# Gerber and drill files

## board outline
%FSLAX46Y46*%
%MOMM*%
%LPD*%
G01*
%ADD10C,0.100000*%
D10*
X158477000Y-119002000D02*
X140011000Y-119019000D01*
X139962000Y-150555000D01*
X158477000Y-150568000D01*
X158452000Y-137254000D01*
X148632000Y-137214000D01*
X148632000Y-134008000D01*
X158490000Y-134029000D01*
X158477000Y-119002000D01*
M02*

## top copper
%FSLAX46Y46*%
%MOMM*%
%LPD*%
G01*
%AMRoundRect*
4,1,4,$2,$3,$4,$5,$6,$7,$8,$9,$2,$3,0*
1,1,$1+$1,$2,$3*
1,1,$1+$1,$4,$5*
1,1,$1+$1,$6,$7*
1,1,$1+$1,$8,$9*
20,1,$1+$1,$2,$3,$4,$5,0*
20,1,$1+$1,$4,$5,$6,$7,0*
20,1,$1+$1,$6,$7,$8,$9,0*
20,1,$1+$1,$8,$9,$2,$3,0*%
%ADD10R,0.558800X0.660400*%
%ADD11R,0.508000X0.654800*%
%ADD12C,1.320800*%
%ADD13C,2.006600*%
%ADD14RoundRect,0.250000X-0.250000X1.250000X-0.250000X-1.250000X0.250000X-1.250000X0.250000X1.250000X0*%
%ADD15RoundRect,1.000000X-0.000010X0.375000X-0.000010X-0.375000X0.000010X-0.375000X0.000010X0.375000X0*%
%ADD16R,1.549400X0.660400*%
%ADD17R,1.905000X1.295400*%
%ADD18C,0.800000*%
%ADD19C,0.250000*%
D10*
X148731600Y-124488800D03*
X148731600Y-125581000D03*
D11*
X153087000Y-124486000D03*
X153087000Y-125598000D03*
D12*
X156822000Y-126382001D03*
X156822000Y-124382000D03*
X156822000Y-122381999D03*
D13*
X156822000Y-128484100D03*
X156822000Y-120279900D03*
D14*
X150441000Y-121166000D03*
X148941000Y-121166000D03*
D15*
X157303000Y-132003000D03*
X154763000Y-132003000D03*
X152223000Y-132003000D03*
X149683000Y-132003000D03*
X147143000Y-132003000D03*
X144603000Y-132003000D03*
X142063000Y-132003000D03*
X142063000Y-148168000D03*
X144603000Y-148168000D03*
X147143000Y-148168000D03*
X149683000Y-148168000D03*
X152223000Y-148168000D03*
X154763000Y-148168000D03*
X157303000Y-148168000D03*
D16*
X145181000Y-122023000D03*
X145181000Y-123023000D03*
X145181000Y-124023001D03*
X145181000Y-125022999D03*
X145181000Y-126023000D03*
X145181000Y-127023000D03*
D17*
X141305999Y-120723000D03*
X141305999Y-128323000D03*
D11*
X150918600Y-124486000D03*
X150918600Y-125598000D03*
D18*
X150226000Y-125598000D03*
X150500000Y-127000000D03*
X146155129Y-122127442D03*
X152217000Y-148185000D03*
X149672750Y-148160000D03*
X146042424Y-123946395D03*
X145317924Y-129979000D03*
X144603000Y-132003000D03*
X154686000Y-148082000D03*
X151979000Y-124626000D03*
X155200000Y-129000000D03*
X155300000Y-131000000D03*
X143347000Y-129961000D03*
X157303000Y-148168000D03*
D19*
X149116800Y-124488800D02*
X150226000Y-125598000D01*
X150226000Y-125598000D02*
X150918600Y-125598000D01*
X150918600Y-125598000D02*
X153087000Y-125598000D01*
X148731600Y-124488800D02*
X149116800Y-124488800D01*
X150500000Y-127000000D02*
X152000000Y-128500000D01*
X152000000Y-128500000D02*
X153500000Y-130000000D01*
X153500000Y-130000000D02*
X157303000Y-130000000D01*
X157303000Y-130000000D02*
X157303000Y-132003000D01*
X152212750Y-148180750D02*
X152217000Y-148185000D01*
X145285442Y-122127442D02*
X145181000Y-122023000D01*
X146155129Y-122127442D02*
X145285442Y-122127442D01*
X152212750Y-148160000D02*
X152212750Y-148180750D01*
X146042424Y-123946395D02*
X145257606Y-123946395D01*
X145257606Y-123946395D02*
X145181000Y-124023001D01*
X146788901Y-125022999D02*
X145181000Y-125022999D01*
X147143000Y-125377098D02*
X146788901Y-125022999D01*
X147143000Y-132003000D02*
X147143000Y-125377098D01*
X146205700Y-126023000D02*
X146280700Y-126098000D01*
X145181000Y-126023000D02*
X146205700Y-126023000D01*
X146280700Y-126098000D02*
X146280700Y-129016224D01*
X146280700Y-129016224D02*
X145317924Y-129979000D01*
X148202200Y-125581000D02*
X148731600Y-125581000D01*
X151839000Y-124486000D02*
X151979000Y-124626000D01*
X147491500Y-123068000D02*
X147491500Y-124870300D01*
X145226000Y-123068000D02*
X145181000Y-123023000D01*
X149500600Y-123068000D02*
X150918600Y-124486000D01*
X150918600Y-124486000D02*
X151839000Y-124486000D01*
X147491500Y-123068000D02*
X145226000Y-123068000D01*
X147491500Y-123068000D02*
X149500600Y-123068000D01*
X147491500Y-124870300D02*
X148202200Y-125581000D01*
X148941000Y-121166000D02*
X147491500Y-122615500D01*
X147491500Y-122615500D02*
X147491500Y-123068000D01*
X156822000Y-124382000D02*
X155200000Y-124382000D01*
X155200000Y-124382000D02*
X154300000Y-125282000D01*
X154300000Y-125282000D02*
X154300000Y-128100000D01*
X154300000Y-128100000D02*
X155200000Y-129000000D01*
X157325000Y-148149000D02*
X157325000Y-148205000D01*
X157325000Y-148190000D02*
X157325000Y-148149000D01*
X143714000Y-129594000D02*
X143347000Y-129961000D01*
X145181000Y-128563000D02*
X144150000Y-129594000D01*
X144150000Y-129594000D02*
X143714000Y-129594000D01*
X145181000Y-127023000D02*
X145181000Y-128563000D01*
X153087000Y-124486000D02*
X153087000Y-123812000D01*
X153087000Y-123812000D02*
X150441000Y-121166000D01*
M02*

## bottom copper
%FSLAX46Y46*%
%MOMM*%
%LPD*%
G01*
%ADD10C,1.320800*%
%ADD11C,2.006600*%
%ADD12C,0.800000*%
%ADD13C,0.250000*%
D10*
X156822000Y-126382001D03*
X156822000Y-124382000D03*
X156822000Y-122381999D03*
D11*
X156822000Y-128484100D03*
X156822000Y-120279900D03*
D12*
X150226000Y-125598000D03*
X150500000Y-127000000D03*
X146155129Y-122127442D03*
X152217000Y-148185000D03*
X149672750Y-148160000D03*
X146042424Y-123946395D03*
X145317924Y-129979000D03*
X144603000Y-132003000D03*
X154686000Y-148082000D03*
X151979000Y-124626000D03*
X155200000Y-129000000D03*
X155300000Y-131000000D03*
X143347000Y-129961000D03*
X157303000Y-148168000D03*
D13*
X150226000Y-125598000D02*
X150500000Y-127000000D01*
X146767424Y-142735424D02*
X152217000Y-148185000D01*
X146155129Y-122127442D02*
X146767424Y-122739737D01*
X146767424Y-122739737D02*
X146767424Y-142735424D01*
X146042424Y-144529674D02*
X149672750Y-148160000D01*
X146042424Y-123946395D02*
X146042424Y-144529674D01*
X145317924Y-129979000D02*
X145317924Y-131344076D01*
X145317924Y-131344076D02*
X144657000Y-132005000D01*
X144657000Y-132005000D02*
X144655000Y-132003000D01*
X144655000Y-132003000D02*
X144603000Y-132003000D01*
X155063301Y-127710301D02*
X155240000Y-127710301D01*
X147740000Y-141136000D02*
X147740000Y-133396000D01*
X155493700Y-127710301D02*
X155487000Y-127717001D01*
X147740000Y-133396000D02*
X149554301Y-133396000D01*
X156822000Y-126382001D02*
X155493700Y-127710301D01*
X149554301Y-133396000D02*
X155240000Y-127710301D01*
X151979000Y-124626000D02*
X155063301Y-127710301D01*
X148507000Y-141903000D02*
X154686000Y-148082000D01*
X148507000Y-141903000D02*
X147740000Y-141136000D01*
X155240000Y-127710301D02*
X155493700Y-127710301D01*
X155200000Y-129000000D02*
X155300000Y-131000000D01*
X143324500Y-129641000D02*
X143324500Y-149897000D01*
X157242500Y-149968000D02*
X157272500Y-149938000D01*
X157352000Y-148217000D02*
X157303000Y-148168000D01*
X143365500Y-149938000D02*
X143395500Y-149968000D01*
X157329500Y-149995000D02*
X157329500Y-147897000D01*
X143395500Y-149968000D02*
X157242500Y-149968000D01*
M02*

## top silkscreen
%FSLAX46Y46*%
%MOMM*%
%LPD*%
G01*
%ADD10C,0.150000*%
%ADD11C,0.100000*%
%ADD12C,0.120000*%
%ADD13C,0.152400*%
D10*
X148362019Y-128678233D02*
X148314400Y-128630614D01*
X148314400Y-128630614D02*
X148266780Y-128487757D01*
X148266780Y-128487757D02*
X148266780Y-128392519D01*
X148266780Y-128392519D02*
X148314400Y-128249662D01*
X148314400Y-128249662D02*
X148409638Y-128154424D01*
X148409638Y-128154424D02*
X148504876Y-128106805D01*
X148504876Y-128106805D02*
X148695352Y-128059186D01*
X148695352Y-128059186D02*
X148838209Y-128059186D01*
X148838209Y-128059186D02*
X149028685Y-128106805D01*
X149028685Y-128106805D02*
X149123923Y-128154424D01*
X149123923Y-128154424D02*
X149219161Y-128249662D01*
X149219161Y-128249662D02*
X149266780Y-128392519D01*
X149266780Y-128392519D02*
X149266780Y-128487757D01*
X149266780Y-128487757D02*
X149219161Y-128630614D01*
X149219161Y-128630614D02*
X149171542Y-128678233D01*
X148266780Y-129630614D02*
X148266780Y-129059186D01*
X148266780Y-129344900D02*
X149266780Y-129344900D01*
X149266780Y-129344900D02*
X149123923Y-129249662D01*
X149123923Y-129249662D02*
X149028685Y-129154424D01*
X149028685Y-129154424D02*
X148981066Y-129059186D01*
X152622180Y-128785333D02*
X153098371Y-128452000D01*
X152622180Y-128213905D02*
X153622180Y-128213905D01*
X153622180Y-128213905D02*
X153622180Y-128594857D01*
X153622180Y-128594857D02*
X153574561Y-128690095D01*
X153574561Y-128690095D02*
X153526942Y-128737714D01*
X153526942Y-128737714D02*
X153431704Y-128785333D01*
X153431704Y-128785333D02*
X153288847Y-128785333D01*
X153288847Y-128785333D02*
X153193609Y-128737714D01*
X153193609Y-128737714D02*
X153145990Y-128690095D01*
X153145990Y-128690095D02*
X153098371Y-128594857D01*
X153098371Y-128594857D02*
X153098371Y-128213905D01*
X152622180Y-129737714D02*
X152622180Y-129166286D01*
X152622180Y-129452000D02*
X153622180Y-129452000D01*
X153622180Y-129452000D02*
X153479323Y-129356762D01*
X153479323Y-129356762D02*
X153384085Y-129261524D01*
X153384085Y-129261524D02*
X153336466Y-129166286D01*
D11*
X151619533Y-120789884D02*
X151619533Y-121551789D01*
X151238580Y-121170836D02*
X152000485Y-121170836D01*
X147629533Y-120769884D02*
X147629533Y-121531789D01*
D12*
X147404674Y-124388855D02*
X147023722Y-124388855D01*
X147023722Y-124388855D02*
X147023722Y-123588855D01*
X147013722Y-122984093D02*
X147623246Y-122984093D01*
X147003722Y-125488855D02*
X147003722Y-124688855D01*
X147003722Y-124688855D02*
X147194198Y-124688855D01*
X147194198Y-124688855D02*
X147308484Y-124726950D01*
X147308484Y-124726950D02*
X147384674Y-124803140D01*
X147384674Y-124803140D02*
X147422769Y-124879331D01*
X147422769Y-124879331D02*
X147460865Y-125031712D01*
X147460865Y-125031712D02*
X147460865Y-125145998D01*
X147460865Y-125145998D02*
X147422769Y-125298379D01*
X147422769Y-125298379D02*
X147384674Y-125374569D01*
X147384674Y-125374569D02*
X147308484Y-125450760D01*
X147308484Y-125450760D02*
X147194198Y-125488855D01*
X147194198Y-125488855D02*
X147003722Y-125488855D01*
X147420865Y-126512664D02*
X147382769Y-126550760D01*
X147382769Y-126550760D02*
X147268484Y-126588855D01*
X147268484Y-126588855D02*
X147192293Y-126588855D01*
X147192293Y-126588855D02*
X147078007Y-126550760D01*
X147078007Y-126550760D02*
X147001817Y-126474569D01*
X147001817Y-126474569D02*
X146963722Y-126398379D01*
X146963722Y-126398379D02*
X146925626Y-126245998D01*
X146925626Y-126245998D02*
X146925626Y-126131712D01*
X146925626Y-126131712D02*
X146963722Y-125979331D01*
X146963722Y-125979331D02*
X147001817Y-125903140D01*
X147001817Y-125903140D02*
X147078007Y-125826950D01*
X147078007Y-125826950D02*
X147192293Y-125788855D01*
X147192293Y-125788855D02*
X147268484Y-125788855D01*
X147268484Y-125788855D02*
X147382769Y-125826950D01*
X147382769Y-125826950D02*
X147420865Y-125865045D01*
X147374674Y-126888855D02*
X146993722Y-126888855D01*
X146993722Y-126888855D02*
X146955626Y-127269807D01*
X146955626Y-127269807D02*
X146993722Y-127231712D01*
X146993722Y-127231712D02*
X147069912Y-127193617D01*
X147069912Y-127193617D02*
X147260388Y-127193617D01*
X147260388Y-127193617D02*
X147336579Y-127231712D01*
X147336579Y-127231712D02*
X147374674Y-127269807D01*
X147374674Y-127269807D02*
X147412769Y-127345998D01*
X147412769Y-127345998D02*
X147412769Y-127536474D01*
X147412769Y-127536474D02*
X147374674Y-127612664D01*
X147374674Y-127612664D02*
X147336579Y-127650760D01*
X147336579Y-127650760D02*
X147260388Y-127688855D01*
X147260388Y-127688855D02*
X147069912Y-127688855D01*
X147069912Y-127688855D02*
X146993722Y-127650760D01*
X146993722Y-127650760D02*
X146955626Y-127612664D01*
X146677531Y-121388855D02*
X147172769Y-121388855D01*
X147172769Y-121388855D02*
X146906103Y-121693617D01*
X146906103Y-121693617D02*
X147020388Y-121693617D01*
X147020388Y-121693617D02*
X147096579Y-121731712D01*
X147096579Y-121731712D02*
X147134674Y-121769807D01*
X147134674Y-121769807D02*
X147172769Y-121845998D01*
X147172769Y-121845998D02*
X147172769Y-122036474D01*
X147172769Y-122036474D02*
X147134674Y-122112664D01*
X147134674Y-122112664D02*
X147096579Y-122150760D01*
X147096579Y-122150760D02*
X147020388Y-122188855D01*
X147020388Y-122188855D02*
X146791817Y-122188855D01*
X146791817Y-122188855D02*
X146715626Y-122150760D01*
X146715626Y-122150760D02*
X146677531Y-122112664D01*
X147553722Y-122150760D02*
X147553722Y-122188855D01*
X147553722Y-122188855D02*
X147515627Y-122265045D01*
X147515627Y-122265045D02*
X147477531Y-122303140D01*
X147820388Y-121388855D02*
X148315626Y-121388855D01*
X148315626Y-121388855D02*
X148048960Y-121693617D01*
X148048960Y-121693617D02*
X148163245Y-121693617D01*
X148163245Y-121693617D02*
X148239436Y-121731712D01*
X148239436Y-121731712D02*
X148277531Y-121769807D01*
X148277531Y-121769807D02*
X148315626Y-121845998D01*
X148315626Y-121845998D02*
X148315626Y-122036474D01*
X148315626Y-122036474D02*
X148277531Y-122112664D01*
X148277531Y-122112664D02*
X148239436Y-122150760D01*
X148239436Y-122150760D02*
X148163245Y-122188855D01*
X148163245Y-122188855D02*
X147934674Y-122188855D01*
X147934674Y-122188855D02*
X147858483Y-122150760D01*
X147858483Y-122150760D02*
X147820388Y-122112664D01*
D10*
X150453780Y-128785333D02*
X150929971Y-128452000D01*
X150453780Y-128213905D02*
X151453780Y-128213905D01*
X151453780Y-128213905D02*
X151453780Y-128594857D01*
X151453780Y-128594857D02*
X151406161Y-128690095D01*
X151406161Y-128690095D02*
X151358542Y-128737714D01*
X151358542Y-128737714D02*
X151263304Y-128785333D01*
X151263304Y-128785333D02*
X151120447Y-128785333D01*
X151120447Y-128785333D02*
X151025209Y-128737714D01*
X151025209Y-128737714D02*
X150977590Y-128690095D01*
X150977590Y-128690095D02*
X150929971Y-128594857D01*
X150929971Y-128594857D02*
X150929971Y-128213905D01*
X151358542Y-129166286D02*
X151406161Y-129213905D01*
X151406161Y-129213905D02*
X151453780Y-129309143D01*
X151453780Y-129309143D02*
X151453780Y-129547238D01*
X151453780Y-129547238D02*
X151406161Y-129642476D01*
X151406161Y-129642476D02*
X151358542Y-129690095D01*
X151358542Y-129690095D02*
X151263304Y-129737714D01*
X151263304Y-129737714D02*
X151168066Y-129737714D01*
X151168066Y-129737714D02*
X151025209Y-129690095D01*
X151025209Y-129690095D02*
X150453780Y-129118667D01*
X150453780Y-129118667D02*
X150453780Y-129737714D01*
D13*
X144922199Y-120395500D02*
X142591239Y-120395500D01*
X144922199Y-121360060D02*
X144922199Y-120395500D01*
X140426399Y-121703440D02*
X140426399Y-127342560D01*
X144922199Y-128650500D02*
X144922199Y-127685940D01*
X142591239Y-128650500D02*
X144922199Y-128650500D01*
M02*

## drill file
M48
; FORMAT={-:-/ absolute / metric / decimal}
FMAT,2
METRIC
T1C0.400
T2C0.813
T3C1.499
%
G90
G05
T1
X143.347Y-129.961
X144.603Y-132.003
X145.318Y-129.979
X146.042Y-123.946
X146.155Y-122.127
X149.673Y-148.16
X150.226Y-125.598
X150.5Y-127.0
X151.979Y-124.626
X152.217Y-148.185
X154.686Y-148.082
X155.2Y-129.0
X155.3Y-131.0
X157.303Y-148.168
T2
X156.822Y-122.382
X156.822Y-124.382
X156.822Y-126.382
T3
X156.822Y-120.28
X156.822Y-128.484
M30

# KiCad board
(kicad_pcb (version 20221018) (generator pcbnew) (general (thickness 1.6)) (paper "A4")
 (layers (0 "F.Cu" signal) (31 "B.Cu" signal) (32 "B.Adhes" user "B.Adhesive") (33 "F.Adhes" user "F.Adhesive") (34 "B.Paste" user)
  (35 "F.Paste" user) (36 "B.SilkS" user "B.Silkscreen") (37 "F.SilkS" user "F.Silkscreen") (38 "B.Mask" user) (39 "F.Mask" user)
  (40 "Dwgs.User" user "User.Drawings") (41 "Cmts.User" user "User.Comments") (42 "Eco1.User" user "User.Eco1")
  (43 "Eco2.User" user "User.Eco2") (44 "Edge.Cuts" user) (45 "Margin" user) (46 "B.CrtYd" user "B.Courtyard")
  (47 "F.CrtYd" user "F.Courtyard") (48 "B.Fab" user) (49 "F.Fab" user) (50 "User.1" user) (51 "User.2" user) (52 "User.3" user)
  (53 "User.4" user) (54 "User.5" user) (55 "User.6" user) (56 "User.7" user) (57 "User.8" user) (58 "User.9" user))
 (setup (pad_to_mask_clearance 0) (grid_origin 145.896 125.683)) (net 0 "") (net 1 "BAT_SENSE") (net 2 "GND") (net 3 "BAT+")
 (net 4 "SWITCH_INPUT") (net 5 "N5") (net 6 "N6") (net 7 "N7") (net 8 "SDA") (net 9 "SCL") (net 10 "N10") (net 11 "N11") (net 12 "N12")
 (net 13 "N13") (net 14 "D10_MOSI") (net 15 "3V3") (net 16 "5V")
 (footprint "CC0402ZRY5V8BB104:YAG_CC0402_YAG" (layer "F.Cu") (at 148.7316 125.0349 -90)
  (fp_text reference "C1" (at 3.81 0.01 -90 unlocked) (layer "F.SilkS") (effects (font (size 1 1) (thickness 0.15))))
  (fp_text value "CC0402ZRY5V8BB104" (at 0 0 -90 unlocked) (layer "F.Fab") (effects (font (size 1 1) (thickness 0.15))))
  (pad "1" smd rect (at -0.5461 0 270) (size 0.6604 0.5588) (layers "F.Cu" "F.Paste" "F.Mask") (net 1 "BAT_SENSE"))
  (pad "2" smd rect (at 0.5461 0 270) (size 0.6604 0.5588) (layers "F.Cu" "F.Paste" "F.Mask") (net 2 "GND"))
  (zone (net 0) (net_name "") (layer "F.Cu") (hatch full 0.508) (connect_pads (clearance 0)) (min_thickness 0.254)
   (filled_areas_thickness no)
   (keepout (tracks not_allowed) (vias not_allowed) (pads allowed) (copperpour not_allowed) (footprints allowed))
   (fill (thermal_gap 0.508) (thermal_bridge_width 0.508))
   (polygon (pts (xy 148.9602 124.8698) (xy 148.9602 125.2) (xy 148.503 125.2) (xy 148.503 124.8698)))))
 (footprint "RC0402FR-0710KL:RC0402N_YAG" (layer "F.Cu") (at 153.087 125.042 -90)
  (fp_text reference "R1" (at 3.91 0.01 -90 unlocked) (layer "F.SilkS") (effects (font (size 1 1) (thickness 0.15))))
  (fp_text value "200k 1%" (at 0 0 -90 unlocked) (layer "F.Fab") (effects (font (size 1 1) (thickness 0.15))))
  (pad "1" smd rect (at -0.556 0 270) (size 0.6548 0.508) (layers "F.Cu" "F.Paste" "F.Mask") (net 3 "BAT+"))
  (pad "2" smd rect (at 0.556 0 270) (size 0.6548 0.508) (layers "F.Cu" "F.Paste" "F.Mask") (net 1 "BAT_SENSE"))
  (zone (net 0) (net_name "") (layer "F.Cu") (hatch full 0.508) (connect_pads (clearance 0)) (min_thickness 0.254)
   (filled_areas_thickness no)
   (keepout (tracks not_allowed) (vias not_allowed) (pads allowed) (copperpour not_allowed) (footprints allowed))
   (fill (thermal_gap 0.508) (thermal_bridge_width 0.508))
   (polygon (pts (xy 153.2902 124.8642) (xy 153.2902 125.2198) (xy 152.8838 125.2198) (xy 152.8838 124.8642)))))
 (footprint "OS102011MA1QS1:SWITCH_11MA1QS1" (layer "F.Cu") (at 156.822 126.382001 90)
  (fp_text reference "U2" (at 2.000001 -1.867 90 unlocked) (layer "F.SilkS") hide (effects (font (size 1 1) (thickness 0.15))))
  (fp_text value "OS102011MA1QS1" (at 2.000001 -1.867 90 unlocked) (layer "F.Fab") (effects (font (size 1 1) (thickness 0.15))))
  (pad "1" thru_hole circle (at 0 0 90) (size 1.3208 1.3208) (drill 0.8128) (layers "*.Cu" "*.Mask") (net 2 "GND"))
  (pad "2" thru_hole circle (at 2.000001 0 90) (size 1.3208 1.3208) (drill 0.8128) (layers "*.Cu" "*.Mask") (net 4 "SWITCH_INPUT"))
  (pad "3" thru_hole circle (at 4.000002 0 90) (size 1.3208 1.3208) (drill 0.8128) (layers "*.Cu" "*.Mask") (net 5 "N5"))
  (pad "4" thru_hole circle (at -2.102099 0 90) (size 2.0066 2.0066) (drill 1.4986) (layers "*.Cu" "*.Mask"))
  (pad "5" thru_hole circle (at 6.102101 0 90) (size 2.0066 2.0066) (drill 1.4986) (layers "*.Cu" "*.Mask")))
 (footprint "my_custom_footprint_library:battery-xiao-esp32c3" (layer "F.Cu") (at 150.941 121.166 -90)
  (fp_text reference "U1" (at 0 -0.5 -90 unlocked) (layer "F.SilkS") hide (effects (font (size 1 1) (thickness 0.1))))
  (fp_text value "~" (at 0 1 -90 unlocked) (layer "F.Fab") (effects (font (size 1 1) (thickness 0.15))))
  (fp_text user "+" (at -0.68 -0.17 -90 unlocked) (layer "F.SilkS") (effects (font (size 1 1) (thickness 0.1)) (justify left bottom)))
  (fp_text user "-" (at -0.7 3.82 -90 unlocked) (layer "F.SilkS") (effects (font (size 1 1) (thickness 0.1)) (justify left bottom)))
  (pad "1" smd roundrect (at 0 0.5 270) (size 3 1) (layers "F.Cu" "F.Paste" "F.Mask") (roundrect_rratio 0.25) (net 3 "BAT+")
   (thermal_bridge_angle 45))
  (pad "2" smd roundrect (at 0 2 270) (size 3 1) (layers "F.Cu" "F.Paste" "F.Mask") (roundrect_rratio 0.25) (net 2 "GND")
   (thermal_bridge_angle 45)))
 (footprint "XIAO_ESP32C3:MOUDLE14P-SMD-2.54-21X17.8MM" (layer "F.Cu") (at 139.183 131.168 -90)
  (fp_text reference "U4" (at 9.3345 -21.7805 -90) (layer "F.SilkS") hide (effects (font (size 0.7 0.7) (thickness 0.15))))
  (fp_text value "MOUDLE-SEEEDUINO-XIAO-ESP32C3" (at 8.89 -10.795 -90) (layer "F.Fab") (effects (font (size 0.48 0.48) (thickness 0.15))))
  (pad "1" smd roundrect (at 0.835 -18.12 270) (size 2.75 2) (layers "F.Cu" "F.Paste" "F.Mask") (roundrect_rratio 0.5) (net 1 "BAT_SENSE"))
  (pad "2" smd roundrect (at 0.835 -15.58 270) (size 2.75 2) (layers "F.Cu" "F.Paste" "F.Mask") (roundrect_rratio 0.5)
   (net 4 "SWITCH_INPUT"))
  (pad "3" smd roundrect (at 0.835 -13.04 270) (size 2.75 2) (layers "F.Cu" "F.Paste" "F.Mask") (roundrect_rratio 0.5) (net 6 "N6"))
  (pad "4" smd roundrect (at 0.835 -10.5 270) (size 2.75 2) (layers "F.Cu" "F.Paste" "F.Mask") (roundrect_rratio 0.5) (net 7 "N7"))
  (pad "5" smd roundrect (at 0.835 -7.96 270) (size 2.75 2) (layers "F.Cu" "F.Paste" "F.Mask") (roundrect_rratio 0.5) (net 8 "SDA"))
  (pad "6" smd roundrect (at 0.835 -5.42 270) (size 2.75 2) (layers "F.Cu" "F.Paste" "F.Mask") (roundrect_rratio 0.5) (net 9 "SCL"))
  (pad "7" smd roundrect (at 0.835 -2.88 270) (size 2.75 2) (layers "F.Cu" "F.Paste" "F.Mask") (roundrect_rratio 0.5) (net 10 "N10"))
  (pad "8" smd roundrect (at 17 -2.88 270) (size 2.75 2) (layers "F.Cu" "F.Paste" "F.Mask") (roundrect_rratio 0.5) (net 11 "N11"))
  (pad "9" smd roundrect (at 17 -5.42 270) (size 2.75 2) (layers "F.Cu" "F.Paste" "F.Mask") (roundrect_rratio 0.5) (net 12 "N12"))
  (pad "10" smd roundrect (at 17 -7.96 270) (size 2.75 2) (layers "F.Cu" "F.Paste" "F.Mask") (roundrect_rratio 0.5) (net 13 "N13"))
  (pad "11" smd roundrect (at 17 -10.5 270) (size 2.75 2) (layers "F.Cu" "F.Paste" "F.Mask") (roundrect_rratio 0.5) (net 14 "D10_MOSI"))
  (pad "12" smd roundrect (at 17 -13.04 270) (size 2.75 2) (layers "F.Cu" "F.Paste" "F.Mask") (roundrect_rratio 0.5) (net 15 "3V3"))
  (pad "13" smd roundrect (at 17 -15.58 270) (size 2.75 2) (layers "F.Cu" "F.Paste" "F.Mask") (roundrect_rratio 0.5) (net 2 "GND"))
  (pad "14" smd roundrect (at 17 -18.12 270) (size 2.75 2) (layers "F.Cu" "F.Paste" "F.Mask") (roundrect_rratio 0.5) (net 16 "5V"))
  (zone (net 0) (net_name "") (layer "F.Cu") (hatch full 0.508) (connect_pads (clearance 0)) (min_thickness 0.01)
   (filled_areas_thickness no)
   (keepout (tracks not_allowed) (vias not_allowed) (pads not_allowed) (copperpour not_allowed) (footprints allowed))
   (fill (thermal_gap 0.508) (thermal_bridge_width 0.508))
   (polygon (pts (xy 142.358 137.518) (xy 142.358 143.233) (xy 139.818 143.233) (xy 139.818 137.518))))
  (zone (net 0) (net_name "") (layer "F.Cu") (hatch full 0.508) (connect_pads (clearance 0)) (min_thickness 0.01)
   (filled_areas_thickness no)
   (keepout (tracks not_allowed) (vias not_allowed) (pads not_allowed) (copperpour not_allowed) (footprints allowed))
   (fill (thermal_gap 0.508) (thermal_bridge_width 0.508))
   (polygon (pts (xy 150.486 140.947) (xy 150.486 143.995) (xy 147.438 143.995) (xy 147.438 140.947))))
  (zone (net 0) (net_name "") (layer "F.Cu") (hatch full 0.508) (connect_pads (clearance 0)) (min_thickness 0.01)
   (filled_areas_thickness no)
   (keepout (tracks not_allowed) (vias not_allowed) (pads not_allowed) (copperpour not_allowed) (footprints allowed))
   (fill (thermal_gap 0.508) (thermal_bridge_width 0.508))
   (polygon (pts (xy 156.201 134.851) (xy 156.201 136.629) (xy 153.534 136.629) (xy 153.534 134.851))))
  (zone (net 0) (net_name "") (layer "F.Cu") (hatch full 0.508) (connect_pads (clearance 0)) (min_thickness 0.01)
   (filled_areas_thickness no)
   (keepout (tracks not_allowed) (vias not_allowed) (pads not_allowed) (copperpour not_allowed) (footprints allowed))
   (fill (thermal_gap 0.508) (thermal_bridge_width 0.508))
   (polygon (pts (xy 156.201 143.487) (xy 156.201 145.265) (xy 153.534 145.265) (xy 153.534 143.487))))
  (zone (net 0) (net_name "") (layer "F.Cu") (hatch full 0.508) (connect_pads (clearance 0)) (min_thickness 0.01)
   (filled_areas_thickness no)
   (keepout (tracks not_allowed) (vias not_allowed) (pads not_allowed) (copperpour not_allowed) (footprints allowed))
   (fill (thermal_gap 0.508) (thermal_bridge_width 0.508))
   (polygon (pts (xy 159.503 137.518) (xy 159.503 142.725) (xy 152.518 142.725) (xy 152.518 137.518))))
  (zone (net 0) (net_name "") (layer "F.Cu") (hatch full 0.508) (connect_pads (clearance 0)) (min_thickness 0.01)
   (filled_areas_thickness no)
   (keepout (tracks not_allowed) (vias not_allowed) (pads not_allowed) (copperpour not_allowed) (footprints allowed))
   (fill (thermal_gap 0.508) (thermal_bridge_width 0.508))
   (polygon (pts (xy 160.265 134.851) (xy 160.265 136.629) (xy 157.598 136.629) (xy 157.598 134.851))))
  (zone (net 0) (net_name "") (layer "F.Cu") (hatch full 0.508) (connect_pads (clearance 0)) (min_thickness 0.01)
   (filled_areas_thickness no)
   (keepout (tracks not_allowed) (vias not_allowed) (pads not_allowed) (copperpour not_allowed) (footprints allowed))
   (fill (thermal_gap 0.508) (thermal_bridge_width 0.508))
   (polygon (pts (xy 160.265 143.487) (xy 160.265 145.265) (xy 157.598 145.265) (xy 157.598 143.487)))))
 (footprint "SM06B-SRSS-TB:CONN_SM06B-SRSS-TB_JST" (layer "F.Cu") (at 142.674299 124.523 -90)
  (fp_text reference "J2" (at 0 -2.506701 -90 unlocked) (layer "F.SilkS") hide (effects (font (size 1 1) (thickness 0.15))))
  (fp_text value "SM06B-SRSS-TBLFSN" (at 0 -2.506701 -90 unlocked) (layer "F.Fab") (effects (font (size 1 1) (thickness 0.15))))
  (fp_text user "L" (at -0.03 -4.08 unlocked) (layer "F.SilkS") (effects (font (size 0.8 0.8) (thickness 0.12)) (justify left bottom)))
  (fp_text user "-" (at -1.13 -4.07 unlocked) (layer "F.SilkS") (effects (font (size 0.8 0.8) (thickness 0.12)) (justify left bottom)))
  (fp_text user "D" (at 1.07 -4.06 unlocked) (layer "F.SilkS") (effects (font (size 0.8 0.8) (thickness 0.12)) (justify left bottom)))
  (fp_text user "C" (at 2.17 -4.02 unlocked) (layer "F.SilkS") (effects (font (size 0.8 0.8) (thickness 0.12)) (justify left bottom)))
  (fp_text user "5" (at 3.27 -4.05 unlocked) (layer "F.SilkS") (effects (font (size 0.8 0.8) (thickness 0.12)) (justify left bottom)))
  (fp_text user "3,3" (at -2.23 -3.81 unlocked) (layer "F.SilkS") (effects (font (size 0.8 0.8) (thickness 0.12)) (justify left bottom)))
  (fp_line (start -4.1275 -2.2479) (end -4.1275 0.08306) (stroke (width 0.1524) (type solid)) (layer "F.SilkS"))
  (fp_line (start -3.16294 -2.2479) (end -4.1275 -2.2479) (stroke (width 0.1524) (type solid)) (layer "F.SilkS"))
  (fp_line (start -2.81956 2.2479) (end 2.81956 2.2479) (stroke (width 0.1524) (type solid)) (layer "F.SilkS"))
  (fp_line (start 4.1275 -2.2479) (end 3.16294 -2.2479) (stroke (width 0.1524) (type solid)) (layer "F.SilkS"))
  (fp_line (start 4.1275 0.08306) (end 4.1275 -2.2479) (stroke (width 0.1524) (type solid)) (layer "F.SilkS"))
  (pad "1" smd rect (at -2.5 -2.506701 270) (size 0.6604 1.5494) (layers "F.Cu" "F.Paste" "F.Mask") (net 15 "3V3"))
  (pad "2" smd rect (at -1.5 -2.506701 270) (size 0.6604 1.5494) (layers "F.Cu" "F.Paste" "F.Mask") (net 2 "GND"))
  (pad "3" smd rect (at -0.499999 -2.506701 270) (size 0.6604 1.5494) (layers "F.Cu" "F.Paste" "F.Mask") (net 14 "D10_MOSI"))
  (pad "4" smd rect (at 0.499999 -2.506701 270) (size 0.6604 1.5494) (layers "F.Cu" "F.Paste" "F.Mask") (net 8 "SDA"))
  (pad "5" smd rect (at 1.5 -2.506701 270) (size 0.6604 1.5494) (layers "F.Cu" "F.Paste" "F.Mask") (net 9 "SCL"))
  (pad "6" smd rect (at 2.5 -2.506701 270) (size 0.6604 1.5494) (layers "F.Cu" "F.Paste" "F.Mask") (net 16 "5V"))
  (pad "7" smd rect (at -3.8 1.3683) (size 1.905 1.2954) (layers "F.Cu" "F.Paste" "F.Mask"))
  (pad "8" smd rect (at 3.8 1.3683) (size 1.905 1.2954) (layers "F.Cu" "F.Paste" "F.Mask")))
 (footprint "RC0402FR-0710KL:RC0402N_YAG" (layer "F.Cu") (at 150.9186 125.042 -90)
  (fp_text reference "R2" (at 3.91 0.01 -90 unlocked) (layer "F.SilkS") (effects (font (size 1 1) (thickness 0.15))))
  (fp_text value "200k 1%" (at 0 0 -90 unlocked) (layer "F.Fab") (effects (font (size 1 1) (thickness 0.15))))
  (pad "1" smd rect (at -0.556 0 270) (size 0.6548 0.508) (layers "F.Cu" "F.Paste" "F.Mask") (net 2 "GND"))
  (pad "2" smd rect (at 0.556 0 270) (size 0.6548 0.508) (layers "F.Cu" "F.Paste" "F.Mask") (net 1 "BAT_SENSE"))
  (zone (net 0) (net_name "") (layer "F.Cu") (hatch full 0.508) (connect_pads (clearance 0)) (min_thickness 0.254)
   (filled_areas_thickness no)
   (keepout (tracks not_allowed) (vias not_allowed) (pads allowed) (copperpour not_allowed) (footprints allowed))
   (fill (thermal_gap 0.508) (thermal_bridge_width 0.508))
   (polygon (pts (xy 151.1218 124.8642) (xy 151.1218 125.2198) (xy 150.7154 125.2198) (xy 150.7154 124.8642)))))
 (gr_poly
  (pts (xy 158.477 119.002) (xy 140.011 119.019) (xy 139.962 150.555) (xy 158.477 150.568) (xy 158.452 137.254) (xy 148.632 137.214)
   (xy 148.632 134.008) (xy 158.49 134.029))
  (stroke (width 0.1) (type solid)) (fill none) (layer "Edge.Cuts"))
 (segment (start 149.1168 124.4888) (end 150.226 125.598) (width 0.25) (layer "F.Cu") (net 1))
 (segment (start 150.226 125.598) (end 150.9186 125.598) (width 0.25) (layer "F.Cu") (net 1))
 (segment (start 150.9186 125.598) (end 153.087 125.598) (width 0.25) (layer "F.Cu") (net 1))
 (segment (start 148.7316 124.4888) (end 149.1168 124.4888) (width 0.25) (layer "F.Cu") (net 1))
 (segment (start 150.226 125.598) (end 150.5 127) (width 0.25) (layer "B.Cu") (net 1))
 (segment (start 150.5 127) (end 152 128.5) (width 0.25) (layer "F.Cu") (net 1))
 (segment (start 152 128.5) (end 153.5 130) (width 0.25) (layer "F.Cu") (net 1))
 (segment (start 153.5 130) (end 157.303 130) (width 0.25) (layer "F.Cu") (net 1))
 (segment (start 157.303 130) (end 157.303 132.003) (width 0.25) (layer "F.Cu") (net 1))
 (via (at 150.226 125.598) (size 0.8) (drill 0.4) (layers "F.Cu" "B.Cu") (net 1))
 (via (at 150.5 127) (size 0.8) (drill 0.4) (layers "F.Cu" "B.Cu") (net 1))
 (segment (start 152.21275 148.18075) (end 152.217 148.185) (width 0.25) (layer "F.Cu") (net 15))
 (segment (start 145.285442 122.127442) (end 145.181 122.023) (width 0.25) (layer "F.Cu") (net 15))
 (segment (start 146.155129 122.127442) (end 145.285442 122.127442) (width 0.25) (layer "F.Cu") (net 15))
 (segment (start 152.21275 148.16) (end 152.21275 148.18075) (width 0.25) (layer "F.Cu") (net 15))
 (via (at 146.155129 122.127442) (size 0.8) (drill 0.4) (layers "F.Cu" "B.Cu") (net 15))
 (via (at 152.217 148.185) (size 0.8) (drill 0.4) (layers "F.Cu" "B.Cu") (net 15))
 (segment (start 146.767424 142.735424) (end 152.217 148.185) (width 0.25) (layer "B.Cu") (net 15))
 (segment (start 146.155129 122.127442) (end 146.767424 122.739737) (width 0.25) (layer "B.Cu") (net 15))
 (segment (start 146.767424 122.739737) (end 146.767424 142.735424) (width 0.25) (layer "B.Cu") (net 15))
 (segment (start 146.042424 123.946395) (end 145.257606 123.946395) (width 0.25) (layer "F.Cu") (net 14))
 (segment (start 145.257606 123.946395) (end 145.181 124.023001) (width 0.25) (layer "F.Cu") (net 14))
 (via (at 149.67275 148.16) (size 0.8) (drill 0.4) (layers "F.Cu" "B.Cu") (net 14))
 (via (at 146.042424 123.946395) (size 0.8) (drill 0.4) (layers "F.Cu" "B.Cu") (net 14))
 (segment (start 146.042424 144.529674) (end 149.67275 148.16) (width 0.25) (layer "B.Cu") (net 14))
 (segment (start 146.042424 123.946395) (end 146.042424 144.529674) (width 0.25) (layer "B.Cu") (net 14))
 (segment (start 146.788901 125.022999) (end 145.181 125.022999) (width 0.25) (layer "F.Cu") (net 8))
 (segment (start 147.143 125.377098) (end 146.788901 125.022999) (width 0.25) (layer "F.Cu") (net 8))
 (segment (start 147.143 132.003) (end 147.143 125.377098) (width 0.25) (layer "F.Cu") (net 8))
 (segment (start 146.2057 126.023) (end 146.2807 126.098) (width 0.25) (layer "F.Cu") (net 9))
 (segment (start 145.181 126.023) (end 146.2057 126.023) (width 0.25) (layer "F.Cu") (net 9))
 (segment (start 146.2807 126.098) (end 146.2807 129.016224) (width 0.25) (layer "F.Cu") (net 9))
 (segment (start 146.2807 129.016224) (end 145.317924 129.979) (width 0.25) (layer "F.Cu") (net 9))
 (via (at 145.317924 129.979) (size 0.8) (drill 0.4) (layers "F.Cu" "B.Cu") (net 9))
 (via (at 144.603 132.003) (size 0.8) (drill 0.4) (layers "F.Cu" "B.Cu") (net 9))
 (segment (start 145.317924 129.979) (end 145.317924 131.344076) (width 0.25) (layer "B.Cu") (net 9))
 (segment (start 145.317924 131.344076) (end 144.657 132.005) (width 0.25) (layer "B.Cu") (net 9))
 (segment (start 144.657 132.005) (end 144.655 132.003) (width 0.25) (layer "B.Cu") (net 9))
 (segment (start 144.655 132.003) (end 144.603 132.003) (width 0.25) (layer "B.Cu") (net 9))
 (segment (start 148.2022 125.581) (end 148.7316 125.581) (width 0.25) (layer "F.Cu") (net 2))
 (segment (start 151.839 124.486) (end 151.979 124.626) (width 0.25) (layer "F.Cu") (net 2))
 (segment (start 147.4915 123.068) (end 147.4915 124.8703) (width 0.25) (layer "F.Cu") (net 2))
 (segment (start 145.226 123.068) (end 145.181 123.023) (width 0.25) (layer "F.Cu") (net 2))
 (segment (start 149.5006 123.068) (end 150.9186 124.486) (width 0.25) (layer "F.Cu") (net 2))
 (segment (start 150.9186 124.486) (end 151.839 124.486) (width 0.25) (layer "F.Cu") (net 2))
 (segment (start 147.4915 123.068) (end 145.226 123.068) (width 0.25) (layer "F.Cu") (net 2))
 (segment (start 147.4915 123.068) (end 149.5006 123.068) (width 0.25) (layer "F.Cu") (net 2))
 (segment (start 147.4915 124.8703) (end 148.2022 125.581) (width 0.25) (layer "F.Cu") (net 2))
 (via (at 154.686 148.082) (size 0.8) (drill 0.4) (layers "F.Cu" "B.Cu") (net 2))
 (via (at 151.979 124.626) (size 0.8) (drill 0.4) (layers "F.Cu" "B.Cu") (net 2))
 (segment (start 155.063301 127.710301) (end 155.24 127.710301) (width 0.25) (layer "B.Cu") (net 2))
 (segment (start 147.74 141.136) (end 147.74 133.396) (width 0.25) (layer "B.Cu") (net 2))
 (segment (start 155.4937 127.710301) (end 155.487 127.717001) (width 0.25) (layer "B.Cu") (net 2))
 (segment (start 147.74 133.396) (end 149.554301 133.396) (width 0.25) (layer "B.Cu") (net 2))
 (segment (start 156.822 126.382001) (end 155.4937 127.710301) (width 0.25) (layer "B.Cu") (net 2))
 (segment (start 149.554301 133.396) (end 155.24 127.710301) (width 0.25) (layer "B.Cu") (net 2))
 (segment (start 151.979 124.626) (end 155.063301 127.710301) (width 0.25) (layer "B.Cu") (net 2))
 (segment (start 148.507 141.903) (end 154.686 148.082) (width 0.25) (layer "B.Cu") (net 2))
 (segment (start 148.507 141.903) (end 147.74 141.136) (width 0.25) (layer "B.Cu") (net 2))
 (segment (start 155.24 127.710301) (end 155.4937 127.710301) (width 0.25) (layer "B.Cu") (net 2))
 (segment (start 148.941 121.166) (end 147.4915 122.6155) (width 0.25) (layer "F.Cu") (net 2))
 (segment (start 147.4915 122.6155) (end 147.4915 123.068) (width 0.25) (layer "F.Cu") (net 2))
 (segment (start 156.822 124.382) (end 155.2 124.382) (width 0.25) (layer "F.Cu") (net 4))
 (segment (start 155.2 124.382) (end 154.3 125.282) (width 0.25) (layer "F.Cu") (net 4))
 (segment (start 154.3 125.282) (end 154.3 128.1) (width 0.25) (layer "F.Cu") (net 4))
 (segment (start 154.3 128.1) (end 155.2 129) (width 0.25) (layer "F.Cu") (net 4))
 (segment (start 155.2 129) (end 155.3 131) (width 0.25) (layer "B.Cu") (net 4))
 (via (at 155.2 129) (size 0.8) (drill 0.4) (layers "F.Cu" "B.Cu") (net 4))
 (via (at 155.3 131) (size 0.8) (drill 0.4) (layers "F.Cu" "B.Cu") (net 4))
 (segment (start 157.325 148.149) (end 157.325 148.205) (width 0.25) (layer "F.Cu") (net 16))
 (segment (start 157.325 148.19) (end 157.325 148.149) (width 0.25) (layer "F.Cu") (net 16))
 (segment (start 143.714 129.594) (end 143.347 129.961) (width 0.25) (layer "F.Cu") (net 16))
 (segment (start 145.181 128.563) (end 144.15 129.594) (width 0.25) (layer "F.Cu") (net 16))
 (segment (start 144.15 129.594) (end 143.714 129.594) (width 0.25) (layer "F.Cu") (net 16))
 (segment (start 145.181 127.023) (end 145.181 128.563) (width 0.25) (layer "F.Cu") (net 16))
 (via (at 143.347 129.961) (size 0.8) (drill 0.4) (layers "F.Cu" "B.Cu") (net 16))
 (via (at 157.303 148.168) (size 0.8) (drill 0.4) (layers "F.Cu" "B.Cu") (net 16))
 (segment (start 143.3245 129.641) (end 143.3245 149.897) (width 0.25) (layer "B.Cu") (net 16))
 (segment (start 157.2425 149.968) (end 157.2725 149.938) (width 0.25) (layer "B.Cu") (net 16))
 (segment (start 157.352 148.217) (end 157.303 148.168) (width 0.25) (layer "B.Cu") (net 16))
 (segment (start 143.3655 149.938) (end 143.3955 149.968) (width 0.25) (layer "B.Cu") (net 16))
 (segment (start 157.3295 149.995) (end 157.3295 147.897) (width 0.25) (layer "B.Cu") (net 16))
 (segment (start 143.3955 149.968) (end 157.2425 149.968) (width 0.25) (layer "B.Cu") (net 16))
 (segment (start 153.087 124.486) (end 153.087 123.812) (width 0.25) (layer "F.Cu") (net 3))
 (segment (start 153.087 123.812) (end 150.441 121.166) (width 0.25) (layer "F.Cu") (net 3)))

